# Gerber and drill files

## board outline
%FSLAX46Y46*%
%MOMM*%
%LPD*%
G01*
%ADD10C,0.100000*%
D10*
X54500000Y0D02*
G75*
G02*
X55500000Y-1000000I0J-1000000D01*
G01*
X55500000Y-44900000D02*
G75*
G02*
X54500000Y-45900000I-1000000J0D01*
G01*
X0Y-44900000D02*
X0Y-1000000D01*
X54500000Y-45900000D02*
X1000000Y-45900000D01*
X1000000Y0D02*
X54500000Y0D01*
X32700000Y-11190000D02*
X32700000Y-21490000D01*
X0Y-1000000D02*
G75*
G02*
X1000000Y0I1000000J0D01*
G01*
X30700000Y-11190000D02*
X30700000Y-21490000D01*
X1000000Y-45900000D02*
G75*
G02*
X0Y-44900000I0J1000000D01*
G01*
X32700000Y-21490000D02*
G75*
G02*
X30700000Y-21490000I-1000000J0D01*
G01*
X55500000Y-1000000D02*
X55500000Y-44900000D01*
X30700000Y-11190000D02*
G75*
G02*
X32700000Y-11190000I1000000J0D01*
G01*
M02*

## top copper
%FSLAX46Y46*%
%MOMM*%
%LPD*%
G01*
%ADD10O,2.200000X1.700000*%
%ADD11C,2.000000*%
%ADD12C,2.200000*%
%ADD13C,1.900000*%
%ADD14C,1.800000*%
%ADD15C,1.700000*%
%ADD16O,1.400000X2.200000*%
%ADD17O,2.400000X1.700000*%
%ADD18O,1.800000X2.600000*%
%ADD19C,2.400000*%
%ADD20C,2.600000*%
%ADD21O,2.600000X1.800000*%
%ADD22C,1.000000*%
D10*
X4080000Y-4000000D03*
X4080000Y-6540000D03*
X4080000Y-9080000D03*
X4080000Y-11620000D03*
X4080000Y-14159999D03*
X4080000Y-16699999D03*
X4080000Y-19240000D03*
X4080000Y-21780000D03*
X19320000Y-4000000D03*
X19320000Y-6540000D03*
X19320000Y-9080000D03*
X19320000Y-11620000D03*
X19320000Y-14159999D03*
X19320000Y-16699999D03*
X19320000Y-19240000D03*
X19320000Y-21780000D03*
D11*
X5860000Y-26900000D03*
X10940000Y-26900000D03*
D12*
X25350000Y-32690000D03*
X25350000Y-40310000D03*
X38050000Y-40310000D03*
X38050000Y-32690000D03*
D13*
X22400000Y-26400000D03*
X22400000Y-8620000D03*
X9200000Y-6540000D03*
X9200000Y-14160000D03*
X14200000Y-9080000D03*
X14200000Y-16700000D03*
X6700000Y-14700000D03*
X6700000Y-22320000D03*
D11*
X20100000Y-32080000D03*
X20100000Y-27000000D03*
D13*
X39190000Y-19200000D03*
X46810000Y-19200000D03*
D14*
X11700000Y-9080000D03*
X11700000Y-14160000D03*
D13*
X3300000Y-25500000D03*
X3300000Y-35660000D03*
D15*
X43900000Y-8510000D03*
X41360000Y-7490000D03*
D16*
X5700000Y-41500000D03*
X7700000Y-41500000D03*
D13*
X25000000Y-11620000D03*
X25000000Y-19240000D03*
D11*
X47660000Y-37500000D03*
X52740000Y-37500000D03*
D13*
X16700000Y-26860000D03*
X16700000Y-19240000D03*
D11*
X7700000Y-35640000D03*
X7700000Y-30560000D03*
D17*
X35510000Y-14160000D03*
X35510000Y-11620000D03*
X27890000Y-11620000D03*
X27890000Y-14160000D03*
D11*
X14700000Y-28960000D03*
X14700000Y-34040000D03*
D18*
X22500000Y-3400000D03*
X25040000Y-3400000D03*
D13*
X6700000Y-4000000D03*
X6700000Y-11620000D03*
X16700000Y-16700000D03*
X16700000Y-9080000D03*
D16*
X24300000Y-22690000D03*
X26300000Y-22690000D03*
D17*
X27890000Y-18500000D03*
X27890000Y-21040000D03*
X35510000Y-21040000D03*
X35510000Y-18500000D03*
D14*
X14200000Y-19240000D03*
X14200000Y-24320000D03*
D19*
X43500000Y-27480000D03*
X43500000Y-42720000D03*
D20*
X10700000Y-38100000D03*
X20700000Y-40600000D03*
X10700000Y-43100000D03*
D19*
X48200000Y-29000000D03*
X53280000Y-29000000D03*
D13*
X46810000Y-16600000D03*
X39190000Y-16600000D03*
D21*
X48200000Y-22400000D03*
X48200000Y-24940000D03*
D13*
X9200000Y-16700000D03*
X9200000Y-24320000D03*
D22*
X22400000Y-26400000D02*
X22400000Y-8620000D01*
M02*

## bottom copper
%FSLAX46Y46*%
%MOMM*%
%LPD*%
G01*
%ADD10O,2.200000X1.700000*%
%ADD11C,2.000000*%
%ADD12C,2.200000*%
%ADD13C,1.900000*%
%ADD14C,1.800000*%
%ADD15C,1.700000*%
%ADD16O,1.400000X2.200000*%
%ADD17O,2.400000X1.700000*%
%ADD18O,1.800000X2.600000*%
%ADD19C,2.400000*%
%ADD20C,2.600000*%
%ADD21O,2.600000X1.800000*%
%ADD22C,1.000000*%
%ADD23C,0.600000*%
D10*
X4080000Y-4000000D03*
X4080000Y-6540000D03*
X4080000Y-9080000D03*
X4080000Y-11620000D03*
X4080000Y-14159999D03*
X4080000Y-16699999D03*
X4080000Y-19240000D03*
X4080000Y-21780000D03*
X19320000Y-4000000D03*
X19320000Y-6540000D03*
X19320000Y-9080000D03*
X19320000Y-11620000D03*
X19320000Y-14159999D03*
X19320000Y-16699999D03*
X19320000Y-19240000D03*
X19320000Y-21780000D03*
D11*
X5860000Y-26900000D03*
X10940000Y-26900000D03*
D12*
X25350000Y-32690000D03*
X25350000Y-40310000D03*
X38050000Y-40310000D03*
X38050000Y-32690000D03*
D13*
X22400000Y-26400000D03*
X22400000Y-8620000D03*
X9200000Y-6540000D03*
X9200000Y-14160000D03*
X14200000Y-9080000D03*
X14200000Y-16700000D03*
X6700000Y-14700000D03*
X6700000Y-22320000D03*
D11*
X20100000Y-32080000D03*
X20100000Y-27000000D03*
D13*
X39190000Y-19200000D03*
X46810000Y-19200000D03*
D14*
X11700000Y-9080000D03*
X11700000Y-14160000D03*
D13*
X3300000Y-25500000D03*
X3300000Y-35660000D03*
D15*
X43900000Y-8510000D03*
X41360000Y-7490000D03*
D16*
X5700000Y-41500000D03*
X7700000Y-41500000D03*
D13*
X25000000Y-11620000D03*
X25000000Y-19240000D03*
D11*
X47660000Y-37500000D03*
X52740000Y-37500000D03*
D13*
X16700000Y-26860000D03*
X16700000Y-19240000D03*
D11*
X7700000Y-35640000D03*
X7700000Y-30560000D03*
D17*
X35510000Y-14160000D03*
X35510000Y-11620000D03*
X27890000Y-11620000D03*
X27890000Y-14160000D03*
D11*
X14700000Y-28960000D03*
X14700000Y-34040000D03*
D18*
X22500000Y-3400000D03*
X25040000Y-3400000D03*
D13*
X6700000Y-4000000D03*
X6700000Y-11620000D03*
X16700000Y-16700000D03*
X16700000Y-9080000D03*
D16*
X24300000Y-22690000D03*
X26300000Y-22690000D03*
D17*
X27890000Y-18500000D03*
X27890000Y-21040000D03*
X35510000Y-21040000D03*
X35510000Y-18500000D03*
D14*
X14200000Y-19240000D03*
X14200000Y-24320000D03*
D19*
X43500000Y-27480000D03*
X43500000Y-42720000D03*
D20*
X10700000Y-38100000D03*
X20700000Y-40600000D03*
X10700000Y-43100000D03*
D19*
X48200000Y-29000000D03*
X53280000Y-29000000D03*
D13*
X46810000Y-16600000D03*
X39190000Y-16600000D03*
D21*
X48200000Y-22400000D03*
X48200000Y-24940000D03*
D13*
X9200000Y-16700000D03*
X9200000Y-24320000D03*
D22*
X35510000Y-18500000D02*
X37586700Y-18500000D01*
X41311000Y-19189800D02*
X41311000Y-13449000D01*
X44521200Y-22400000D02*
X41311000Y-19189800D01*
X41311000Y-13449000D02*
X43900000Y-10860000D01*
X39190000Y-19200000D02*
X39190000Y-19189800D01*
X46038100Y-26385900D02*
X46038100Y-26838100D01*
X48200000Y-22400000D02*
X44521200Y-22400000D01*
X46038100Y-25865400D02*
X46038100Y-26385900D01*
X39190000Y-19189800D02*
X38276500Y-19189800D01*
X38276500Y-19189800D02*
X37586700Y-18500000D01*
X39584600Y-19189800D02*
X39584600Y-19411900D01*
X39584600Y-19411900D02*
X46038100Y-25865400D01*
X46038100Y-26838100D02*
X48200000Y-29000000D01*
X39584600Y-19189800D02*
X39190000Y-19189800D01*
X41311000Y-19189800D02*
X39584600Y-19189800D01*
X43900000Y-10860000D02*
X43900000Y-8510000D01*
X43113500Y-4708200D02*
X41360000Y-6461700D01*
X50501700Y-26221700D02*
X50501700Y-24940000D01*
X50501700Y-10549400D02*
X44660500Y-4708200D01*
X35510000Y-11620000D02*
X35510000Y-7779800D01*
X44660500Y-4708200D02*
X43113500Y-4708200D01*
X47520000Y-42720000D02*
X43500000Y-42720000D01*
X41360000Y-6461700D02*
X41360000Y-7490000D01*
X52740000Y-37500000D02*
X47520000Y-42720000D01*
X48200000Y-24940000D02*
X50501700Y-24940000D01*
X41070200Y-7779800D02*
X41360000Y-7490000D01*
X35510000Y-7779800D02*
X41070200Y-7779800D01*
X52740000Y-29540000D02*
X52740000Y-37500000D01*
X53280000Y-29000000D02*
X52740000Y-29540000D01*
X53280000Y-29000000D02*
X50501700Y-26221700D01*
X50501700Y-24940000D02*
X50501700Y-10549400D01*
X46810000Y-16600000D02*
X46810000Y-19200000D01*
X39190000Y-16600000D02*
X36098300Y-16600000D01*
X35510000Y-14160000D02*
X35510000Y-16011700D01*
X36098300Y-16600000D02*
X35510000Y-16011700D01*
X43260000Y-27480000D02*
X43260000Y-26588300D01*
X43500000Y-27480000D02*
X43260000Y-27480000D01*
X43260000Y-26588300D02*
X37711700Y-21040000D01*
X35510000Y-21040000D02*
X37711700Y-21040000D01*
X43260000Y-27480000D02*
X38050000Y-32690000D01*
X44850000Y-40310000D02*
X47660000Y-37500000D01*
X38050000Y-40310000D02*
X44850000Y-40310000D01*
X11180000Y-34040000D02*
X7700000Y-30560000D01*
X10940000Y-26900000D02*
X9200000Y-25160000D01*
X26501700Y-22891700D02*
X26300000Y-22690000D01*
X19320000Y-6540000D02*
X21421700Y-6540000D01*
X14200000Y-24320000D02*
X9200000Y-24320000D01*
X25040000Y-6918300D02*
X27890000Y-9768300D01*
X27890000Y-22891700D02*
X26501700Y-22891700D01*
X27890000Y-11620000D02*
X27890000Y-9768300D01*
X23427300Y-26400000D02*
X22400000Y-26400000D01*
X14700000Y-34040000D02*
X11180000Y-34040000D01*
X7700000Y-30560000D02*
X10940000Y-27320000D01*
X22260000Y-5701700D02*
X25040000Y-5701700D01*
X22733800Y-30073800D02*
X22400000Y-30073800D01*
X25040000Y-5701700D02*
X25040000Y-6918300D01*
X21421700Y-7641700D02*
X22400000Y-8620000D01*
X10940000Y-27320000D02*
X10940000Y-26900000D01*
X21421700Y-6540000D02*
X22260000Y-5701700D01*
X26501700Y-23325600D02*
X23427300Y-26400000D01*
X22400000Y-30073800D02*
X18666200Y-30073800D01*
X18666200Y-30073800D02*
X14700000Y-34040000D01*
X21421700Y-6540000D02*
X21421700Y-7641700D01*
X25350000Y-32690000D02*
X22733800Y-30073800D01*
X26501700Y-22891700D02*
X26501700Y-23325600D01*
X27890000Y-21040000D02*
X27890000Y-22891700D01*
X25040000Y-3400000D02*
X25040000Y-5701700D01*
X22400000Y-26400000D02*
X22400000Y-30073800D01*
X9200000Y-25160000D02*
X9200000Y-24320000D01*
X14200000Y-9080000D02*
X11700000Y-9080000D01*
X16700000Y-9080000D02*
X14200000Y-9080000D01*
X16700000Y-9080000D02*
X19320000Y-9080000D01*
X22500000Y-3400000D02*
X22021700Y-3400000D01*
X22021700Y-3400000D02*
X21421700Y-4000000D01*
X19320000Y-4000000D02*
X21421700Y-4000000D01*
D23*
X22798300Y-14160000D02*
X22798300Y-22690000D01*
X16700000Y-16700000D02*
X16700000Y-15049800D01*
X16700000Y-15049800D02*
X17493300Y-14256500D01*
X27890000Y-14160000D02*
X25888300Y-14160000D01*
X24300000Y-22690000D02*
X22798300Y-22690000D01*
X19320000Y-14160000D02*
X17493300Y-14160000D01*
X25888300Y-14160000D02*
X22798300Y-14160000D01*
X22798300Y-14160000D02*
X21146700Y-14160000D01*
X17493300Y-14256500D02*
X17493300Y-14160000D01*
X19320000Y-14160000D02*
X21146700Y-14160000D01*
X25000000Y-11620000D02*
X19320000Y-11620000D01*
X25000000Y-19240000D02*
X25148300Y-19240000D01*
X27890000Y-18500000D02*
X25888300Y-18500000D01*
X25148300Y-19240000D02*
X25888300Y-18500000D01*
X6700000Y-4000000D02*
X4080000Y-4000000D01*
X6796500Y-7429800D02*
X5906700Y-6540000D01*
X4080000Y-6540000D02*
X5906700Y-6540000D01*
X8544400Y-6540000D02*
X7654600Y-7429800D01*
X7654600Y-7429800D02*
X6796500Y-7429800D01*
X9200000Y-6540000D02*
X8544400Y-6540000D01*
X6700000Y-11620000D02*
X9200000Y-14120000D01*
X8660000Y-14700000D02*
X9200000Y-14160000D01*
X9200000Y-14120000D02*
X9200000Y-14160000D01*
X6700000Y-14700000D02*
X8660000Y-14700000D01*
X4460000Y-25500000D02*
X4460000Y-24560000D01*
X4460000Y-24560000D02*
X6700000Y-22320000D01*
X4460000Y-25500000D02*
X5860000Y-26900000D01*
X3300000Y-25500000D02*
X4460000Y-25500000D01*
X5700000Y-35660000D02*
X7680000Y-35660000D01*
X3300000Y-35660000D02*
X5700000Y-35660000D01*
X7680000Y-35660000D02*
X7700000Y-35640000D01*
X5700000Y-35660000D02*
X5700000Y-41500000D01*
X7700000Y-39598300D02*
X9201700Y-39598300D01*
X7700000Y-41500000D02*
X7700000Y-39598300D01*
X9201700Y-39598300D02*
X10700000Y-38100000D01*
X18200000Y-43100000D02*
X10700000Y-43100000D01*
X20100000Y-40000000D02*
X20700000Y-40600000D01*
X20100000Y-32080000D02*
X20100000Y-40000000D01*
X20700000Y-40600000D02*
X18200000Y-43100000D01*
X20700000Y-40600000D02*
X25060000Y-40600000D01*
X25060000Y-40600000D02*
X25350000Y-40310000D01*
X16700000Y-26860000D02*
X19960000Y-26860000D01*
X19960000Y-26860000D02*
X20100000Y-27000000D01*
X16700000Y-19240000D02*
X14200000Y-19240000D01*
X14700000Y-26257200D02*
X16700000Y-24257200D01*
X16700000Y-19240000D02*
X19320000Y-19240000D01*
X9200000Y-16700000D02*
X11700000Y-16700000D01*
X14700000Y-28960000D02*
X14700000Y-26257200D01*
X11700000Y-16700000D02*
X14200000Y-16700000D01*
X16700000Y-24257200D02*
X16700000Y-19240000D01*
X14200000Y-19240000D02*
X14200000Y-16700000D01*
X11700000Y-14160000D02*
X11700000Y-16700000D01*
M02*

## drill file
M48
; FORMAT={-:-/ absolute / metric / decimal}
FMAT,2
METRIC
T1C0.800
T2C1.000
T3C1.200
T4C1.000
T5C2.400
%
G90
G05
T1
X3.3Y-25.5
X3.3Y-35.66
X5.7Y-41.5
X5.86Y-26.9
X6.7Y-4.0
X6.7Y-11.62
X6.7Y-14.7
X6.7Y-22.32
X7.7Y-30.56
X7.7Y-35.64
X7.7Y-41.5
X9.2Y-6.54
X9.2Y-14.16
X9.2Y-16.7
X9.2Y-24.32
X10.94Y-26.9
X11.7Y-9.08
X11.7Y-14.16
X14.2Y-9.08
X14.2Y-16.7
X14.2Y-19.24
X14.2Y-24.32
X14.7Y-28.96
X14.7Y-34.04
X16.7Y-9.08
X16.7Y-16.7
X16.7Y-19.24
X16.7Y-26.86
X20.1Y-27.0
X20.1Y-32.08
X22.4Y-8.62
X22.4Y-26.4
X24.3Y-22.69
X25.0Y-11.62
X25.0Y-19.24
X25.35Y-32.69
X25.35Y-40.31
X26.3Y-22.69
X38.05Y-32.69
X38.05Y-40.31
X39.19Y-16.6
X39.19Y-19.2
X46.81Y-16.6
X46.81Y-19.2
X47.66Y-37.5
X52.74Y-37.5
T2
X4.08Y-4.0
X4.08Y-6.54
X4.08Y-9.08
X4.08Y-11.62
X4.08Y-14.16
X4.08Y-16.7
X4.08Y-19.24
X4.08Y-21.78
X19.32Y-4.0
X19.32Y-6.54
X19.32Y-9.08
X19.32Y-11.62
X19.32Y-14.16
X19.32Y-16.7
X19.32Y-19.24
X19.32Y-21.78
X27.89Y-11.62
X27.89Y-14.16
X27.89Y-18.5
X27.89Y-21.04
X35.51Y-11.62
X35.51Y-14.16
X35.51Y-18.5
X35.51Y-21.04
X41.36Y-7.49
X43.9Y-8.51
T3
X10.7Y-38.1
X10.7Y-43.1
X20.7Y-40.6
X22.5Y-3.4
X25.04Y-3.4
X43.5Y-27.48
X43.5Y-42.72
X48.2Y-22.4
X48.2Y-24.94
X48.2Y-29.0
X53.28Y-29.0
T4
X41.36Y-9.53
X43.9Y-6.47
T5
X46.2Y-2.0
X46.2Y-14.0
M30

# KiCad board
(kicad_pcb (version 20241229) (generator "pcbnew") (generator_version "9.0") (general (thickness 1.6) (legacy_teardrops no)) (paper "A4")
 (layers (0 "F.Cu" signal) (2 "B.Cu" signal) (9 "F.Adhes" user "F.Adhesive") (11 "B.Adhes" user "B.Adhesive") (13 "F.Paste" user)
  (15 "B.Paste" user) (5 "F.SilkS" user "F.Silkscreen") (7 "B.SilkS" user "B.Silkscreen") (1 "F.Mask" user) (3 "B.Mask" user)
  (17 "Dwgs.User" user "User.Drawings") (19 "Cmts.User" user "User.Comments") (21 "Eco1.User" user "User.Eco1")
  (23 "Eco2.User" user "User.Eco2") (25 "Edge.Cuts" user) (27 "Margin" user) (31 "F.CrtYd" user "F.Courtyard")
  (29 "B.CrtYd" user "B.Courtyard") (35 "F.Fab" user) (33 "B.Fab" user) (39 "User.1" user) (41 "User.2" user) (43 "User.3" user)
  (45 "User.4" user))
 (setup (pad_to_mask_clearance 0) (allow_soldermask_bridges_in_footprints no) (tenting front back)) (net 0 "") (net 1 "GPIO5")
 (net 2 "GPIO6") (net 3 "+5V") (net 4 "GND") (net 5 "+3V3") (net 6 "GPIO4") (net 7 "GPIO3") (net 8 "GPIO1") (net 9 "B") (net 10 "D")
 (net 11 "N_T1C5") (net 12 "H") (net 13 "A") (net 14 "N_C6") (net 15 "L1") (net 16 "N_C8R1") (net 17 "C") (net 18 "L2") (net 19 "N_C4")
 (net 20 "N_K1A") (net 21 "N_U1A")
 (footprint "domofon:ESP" (layer "F.Cu") (at 11.7 12.89)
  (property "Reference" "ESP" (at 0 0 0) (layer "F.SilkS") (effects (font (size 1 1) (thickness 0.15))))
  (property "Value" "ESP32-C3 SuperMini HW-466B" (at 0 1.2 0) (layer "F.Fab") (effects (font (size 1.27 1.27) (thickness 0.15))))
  (pad "L1" thru_hole oval (at -7.62 -8.89) (size 2.2 1.7) (drill 1) (layers "B.Cu" "B.Mask") (remove_unused_layers no) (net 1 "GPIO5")
   (thermal_bridge_angle 45))
  (pad "L2" thru_hole oval (at -7.62 -6.35) (size 2.2 1.7) (drill 1) (layers "B.Cu" "B.Mask") (remove_unused_layers no) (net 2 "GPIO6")
   (thermal_bridge_angle 45))
  (pad "L3" thru_hole oval (at -7.62 -3.81) (size 2.2 1.7) (drill 1) (layers "B.Cu" "B.Mask") (remove_unused_layers no)
   (thermal_bridge_angle 45))
  (pad "L4" thru_hole oval (at -7.62 -1.27) (size 2.2 1.7) (drill 1) (layers "B.Cu" "B.Mask") (remove_unused_layers no)
   (thermal_bridge_angle 45))
  (pad "L5" thru_hole oval (at -7.62 1.269999) (size 2.2 1.7) (drill 1) (layers "B.Cu" "B.Mask") (remove_unused_layers no)
   (thermal_bridge_angle 45))
  (pad "L6" thru_hole oval (at -7.62 3.809999) (size 2.2 1.7) (drill 1) (layers "B.Cu" "B.Mask") (remove_unused_layers no)
   (thermal_bridge_angle 45))
  (pad "L7" thru_hole oval (at -7.62 6.35) (size 2.2 1.7) (drill 1) (layers "B.Cu" "B.Mask") (remove_unused_layers no)
   (thermal_bridge_angle 45))
  (pad "L8" thru_hole oval (at -7.62 8.89) (size 2.2 1.7) (drill 1) (layers "B.Cu" "B.Mask") (remove_unused_layers no)
   (thermal_bridge_angle 45))
  (pad "R1" thru_hole oval (at 7.62 -8.89) (size 2.2 1.7) (drill 1) (layers "B.Cu" "B.Mask") (remove_unused_layers no) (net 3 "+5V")
   (thermal_bridge_angle 45))
  (pad "R2" thru_hole oval (at 7.62 -6.35) (size 2.2 1.7) (drill 1) (layers "B.Cu" "B.Mask") (remove_unused_layers no) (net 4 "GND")
   (thermal_bridge_angle 45))
  (pad "R3" thru_hole oval (at 7.62 -3.81) (size 2.2 1.7) (drill 1) (layers "B.Cu" "B.Mask") (remove_unused_layers no) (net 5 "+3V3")
   (thermal_bridge_angle 45))
  (pad "R4" thru_hole oval (at 7.62 -1.27) (size 2.2 1.7) (drill 1) (layers "B.Cu" "B.Mask") (remove_unused_layers no) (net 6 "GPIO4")
   (thermal_bridge_angle 45))
  (pad "R5" thru_hole oval (at 7.62 1.269999) (size 2.2 1.7) (drill 1) (layers "B.Cu" "B.Mask") (remove_unused_layers no) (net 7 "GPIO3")
   (thermal_bridge_angle 45))
  (pad "R6" thru_hole oval (at 7.62 3.809999) (size 2.2 1.7) (drill 1) (layers "B.Cu" "B.Mask") (remove_unused_layers no)
   (thermal_bridge_angle 45))
  (pad "R7" thru_hole oval (at 7.62 6.35) (size 2.2 1.7) (drill 1) (layers "B.Cu" "B.Mask") (remove_unused_layers no) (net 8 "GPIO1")
   (thermal_bridge_angle 45))
  (pad "R8" thru_hole oval (at 7.62 8.89) (size 2.2 1.7) (drill 1) (layers "B.Cu" "B.Mask") (remove_unused_layers no)
   (thermal_bridge_angle 45)))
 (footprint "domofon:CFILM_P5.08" (layer "F.Cu") (at 8.4 26.9)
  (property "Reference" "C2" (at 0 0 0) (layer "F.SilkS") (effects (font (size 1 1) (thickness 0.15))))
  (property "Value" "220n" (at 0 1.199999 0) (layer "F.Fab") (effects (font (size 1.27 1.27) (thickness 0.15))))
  (pad "1" thru_hole circle (at -2.54 0) (size 2 2) (drill 0.8) (layers "B.Cu" "B.Mask") (remove_unused_layers no) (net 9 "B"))
  (pad "2" thru_hole circle (at 2.54 0) (size 2 2) (drill 0.8) (layers "B.Cu" "B.Mask") (remove_unused_layers no) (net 4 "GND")))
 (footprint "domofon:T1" (layer "F.Cu") (at 31.7 36.5)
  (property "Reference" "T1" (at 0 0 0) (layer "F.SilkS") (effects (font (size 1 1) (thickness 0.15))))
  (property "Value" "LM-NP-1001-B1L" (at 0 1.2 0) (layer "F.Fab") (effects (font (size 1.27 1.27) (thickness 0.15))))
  (pad "1" thru_hole circle (at -6.35 -3.81) (size 2.2 2.2) (drill 0.8) (layers "B.Cu" "B.Mask") (remove_unused_layers no) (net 4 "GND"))
  (pad "4" thru_hole circle (at -6.35 3.81) (size 2.2 2.2) (drill 0.8) (layers "B.Cu" "B.Mask") (remove_unused_layers no) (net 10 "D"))
  (pad "5" thru_hole circle (at 6.35 3.81) (size 2.2 2.2) (drill 0.8) (layers "B.Cu" "B.Mask") (remove_unused_layers no) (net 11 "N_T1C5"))
  (pad "8" thru_hole circle (at 6.35 -3.81) (size 2.2 2.2) (drill 0.8) (layers "B.Cu" "B.Mask") (remove_unused_layers no) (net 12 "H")))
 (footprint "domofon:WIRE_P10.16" (layer "F.Cu") (at 22.4 17.51 90)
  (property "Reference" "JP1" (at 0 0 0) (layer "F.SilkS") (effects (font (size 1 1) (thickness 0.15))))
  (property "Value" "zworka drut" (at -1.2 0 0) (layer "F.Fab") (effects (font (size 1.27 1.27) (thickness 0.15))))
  (pad "1" thru_hole circle (at -8.89 0 90) (size 1.9 1.9) (drill 0.8) (layers "*.Cu" "B.Mask") (remove_unused_layers no) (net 4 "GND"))
  (pad "2" thru_hole circle (at 8.89 0 90) (size 1.9 1.9) (drill 0.8) (layers "*.Cu" "B.Mask") (remove_unused_layers no) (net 4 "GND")))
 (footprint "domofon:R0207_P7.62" (layer "F.Cu") (at 9.2 10.35 -90)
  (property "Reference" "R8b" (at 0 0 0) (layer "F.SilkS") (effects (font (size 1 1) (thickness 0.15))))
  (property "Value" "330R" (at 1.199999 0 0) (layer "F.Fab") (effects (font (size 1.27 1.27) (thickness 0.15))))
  (pad "1" thru_hole circle (at -3.81 0 270) (size 1.9 1.9) (drill 0.8) (layers "B.Cu" "B.Mask") (remove_unused_layers no) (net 2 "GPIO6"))
  (pad "2" thru_hole circle (at 3.81 0 270) (size 1.9 1.9) (drill 0.8) (layers "B.Cu" "B.Mask") (remove_unused_layers no) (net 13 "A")))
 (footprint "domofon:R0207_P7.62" (layer "F.Cu") (at 14.2 12.89 -90)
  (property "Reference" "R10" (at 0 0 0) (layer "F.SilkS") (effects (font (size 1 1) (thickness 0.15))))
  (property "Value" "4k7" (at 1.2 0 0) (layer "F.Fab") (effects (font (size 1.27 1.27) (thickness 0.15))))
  (pad "1" thru_hole circle (at -3.81 0 270) (size 1.9 1.9) (drill 0.8) (layers "B.Cu" "B.Mask") (remove_unused_layers no) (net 5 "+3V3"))
  (pad "2" thru_hole circle (at 3.81 0 270) (size 1.9 1.9) (drill 0.8) (layers "B.Cu" "B.Mask") (remove_unused_layers no) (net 8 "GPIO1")))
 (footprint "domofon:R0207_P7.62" (layer "F.Cu") (at 6.7 18.51 -90)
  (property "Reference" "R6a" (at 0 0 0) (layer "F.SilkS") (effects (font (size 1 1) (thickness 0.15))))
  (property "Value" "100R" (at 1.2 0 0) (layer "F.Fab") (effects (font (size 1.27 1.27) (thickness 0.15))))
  (pad "1" thru_hole circle (at -3.81 0 270) (size 1.9 1.9) (drill 0.8) (layers "B.Cu" "B.Mask") (remove_unused_layers no) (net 13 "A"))
  (pad "2" thru_hole circle (at 3.81 0 270) (size 1.9 1.9) (drill 0.8) (layers "B.Cu" "B.Mask") (remove_unused_layers no) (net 9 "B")))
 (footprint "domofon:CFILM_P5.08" (layer "F.Cu") (at 20.1 29.54 90)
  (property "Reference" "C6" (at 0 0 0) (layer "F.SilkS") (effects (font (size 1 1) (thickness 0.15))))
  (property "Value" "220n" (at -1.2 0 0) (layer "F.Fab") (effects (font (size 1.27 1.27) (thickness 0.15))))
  (pad "1" thru_hole circle (at -2.54 0 90) (size 2 2) (drill 0.8) (layers "B.Cu" "B.Mask") (remove_unused_layers no) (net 10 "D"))
  (pad "2" thru_hole circle (at 2.54 0 90) (size 2 2) (drill 0.8) (layers "B.Cu" "B.Mask") (remove_unused_layers no) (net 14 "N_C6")))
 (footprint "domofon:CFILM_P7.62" (layer "F.Cu") (at 43 19.2)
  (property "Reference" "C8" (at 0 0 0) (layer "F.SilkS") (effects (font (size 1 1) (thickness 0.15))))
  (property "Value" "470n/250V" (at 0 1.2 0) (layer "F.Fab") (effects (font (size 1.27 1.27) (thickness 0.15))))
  (pad "1" thru_hole circle (at -3.81 0) (size 1.9 1.9) (drill 0.8) (layers "B.Cu" "B.Mask") (remove_unused_layers no) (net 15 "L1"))
  (pad "2" thru_hole circle (at 3.81 0) (size 1.9 1.9) (drill 0.8) (layers "B.Cu" "B.Mask") (remove_unused_layers no) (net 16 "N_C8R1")))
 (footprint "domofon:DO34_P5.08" (layer "F.Cu") (at 11.7 11.62 -90)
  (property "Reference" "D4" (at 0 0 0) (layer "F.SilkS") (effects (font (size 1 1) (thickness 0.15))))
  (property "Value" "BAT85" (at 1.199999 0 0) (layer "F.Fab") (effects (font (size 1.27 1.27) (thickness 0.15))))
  (pad "1" thru_hole circle (at -2.54 0 270) (size 1.8 1.8) (drill 0.8) (layers "B.Cu" "B.Mask") (remove_unused_layers no) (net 5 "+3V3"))
  (pad "2" thru_hole circle (at 2.54 0 270) (size 1.8 1.8) (drill 0.8) (layers "B.Cu" "B.Mask") (remove_unused_layers no) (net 8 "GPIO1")))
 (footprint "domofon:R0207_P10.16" (layer "F.Cu") (at 3.3 30.58 -90)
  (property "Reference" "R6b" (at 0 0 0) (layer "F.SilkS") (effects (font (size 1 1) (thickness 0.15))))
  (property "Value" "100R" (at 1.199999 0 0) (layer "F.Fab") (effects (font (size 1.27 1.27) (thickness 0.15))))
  (pad "1" thru_hole circle (at -5.08 0 270) (size 1.9 1.9) (drill 0.8) (layers "B.Cu" "B.Mask") (remove_unused_layers no) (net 9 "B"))
  (pad "2" thru_hole circle (at 5.08 0 270) (size 1.9 1.9) (drill 0.8) (layers "B.Cu" "B.Mask") (remove_unused_layers no) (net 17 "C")))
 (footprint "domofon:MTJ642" (layer "F.Cu") (at 46.2 8)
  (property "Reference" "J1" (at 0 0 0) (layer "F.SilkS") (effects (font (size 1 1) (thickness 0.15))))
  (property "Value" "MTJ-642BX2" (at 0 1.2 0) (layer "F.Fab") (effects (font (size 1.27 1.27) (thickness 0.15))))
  (pad "" np_thru_hole circle (at -4.84 1.53) (size 1 1) (drill 1) (layers "B.Cu" "B.Mask"))
  (pad "" np_thru_hole circle (at -2.3 -1.53) (size 1 1) (drill 1) (layers "B.Cu" "B.Mask"))
  (pad "" np_thru_hole circle (at 0 -6) (size 2.4 2.4) (drill 2.4) (layers "B.Cu" "B.Mask"))
  (pad "" np_thru_hole circle (at 0 6) (size 2.4 2.4) (drill 2.4) (layers "B.Cu" "B.Mask"))
  (pad "2" thru_hole circle (at -2.3 0.51) (size 1.7 1.7) (drill 1) (layers "B.Cu" "B.Mask") (remove_unused_layers no) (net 15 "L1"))
  (pad "3" thru_hole circle (at -4.84 -0.51) (size 1.7 1.7) (drill 1) (layers "B.Cu" "B.Mask") (remove_unused_layers no) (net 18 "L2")))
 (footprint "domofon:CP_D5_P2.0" (layer "F.Cu") (at 6.7 41.5)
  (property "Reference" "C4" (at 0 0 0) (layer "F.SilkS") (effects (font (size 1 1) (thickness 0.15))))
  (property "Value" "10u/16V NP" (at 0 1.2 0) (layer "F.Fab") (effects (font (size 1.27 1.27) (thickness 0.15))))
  (pad "1" thru_hole oval (at -1 0) (size 1.4 2.2) (drill 0.8) (layers "B.Cu" "B.Mask") (remove_unused_layers no) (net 17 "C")
   (thermal_bridge_angle 45))
  (pad "2" thru_hole oval (at 1 0) (size 1.4 2.2) (drill 0.8) (layers "B.Cu" "B.Mask") (remove_unused_layers no) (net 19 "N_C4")
   (thermal_bridge_angle 45)))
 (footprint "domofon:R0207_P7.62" (layer "F.Cu") (at 25 15.43 -90)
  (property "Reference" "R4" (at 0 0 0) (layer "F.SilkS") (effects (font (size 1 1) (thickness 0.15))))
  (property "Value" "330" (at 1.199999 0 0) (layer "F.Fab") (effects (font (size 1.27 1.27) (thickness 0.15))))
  (pad "1" thru_hole circle (at -3.81 0 270) (size 1.9 1.9) (drill 0.8) (layers "B.Cu" "B.Mask") (remove_unused_layers no) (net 6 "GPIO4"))
  (pad "2" thru_hole circle (at 3.81 0 270) (size 1.9 1.9) (drill 0.8) (layers "B.Cu" "B.Mask") (remove_unused_layers no) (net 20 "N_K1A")))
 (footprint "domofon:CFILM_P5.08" (layer "F.Cu") (at 50.2 37.5)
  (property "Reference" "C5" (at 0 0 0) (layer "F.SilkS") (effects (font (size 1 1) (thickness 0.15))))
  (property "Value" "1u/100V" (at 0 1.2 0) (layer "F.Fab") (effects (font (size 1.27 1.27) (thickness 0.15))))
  (pad "1" thru_hole circle (at -2.54 0) (size 2 2) (drill 0.8) (layers "B.Cu" "B.Mask") (remove_unused_layers no) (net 11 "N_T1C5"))
  (pad "2" thru_hole circle (at 2.54 0) (size 2 2) (drill 0.8) (layers "B.Cu" "B.Mask") (remove_unused_layers no) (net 18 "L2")))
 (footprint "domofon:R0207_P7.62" (layer "F.Cu") (at 16.7 23.05 90)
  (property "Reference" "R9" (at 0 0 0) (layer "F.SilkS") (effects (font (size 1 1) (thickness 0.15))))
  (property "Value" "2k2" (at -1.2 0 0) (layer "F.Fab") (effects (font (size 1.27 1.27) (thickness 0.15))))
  (pad "1" thru_hole circle (at -3.81 0 90) (size 1.9 1.9) (drill 0.8) (layers "B.Cu" "B.Mask") (remove_unused_layers no) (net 14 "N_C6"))
  (pad "2" thru_hole circle (at 3.81 0 90) (size 1.9 1.9) (drill 0.8) (layers "B.Cu" "B.Mask") (remove_unused_layers no) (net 8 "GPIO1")))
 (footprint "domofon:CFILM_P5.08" (layer "F.Cu") (at 7.7 33.1 90)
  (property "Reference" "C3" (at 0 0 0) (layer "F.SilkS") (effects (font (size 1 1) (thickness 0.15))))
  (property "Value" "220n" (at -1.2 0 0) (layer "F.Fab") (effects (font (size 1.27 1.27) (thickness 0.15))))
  (pad "1" thru_hole circle (at -2.54 0 90) (size 2 2) (drill 0.8) (layers "B.Cu" "B.Mask") (remove_unused_layers no) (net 17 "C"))
  (pad "2" thru_hole circle (at 2.54 0 90) (size 2 2) (drill 0.8) (layers "B.Cu" "B.Mask") (remove_unused_layers no) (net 4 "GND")))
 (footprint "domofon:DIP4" (layer "F.Cu") (at 31.7 12.89 180)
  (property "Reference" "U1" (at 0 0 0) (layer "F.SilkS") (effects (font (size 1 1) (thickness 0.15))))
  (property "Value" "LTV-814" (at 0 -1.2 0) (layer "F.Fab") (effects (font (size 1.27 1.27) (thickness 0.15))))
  (pad "1" thru_hole oval (at -3.81 -1.27 180) (size 2.4 1.7) (drill 1) (layers "B.Cu" "B.Mask") (remove_unused_layers no) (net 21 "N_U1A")
   (thermal_bridge_angle 45))
  (pad "2" thru_hole oval (at -3.81 1.27 180) (size 2.4 1.7) (drill 1) (layers "B.Cu" "B.Mask") (remove_unused_layers no) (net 18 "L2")
   (thermal_bridge_angle 45))
  (pad "3" thru_hole oval (at 3.81 1.27 180) (size 2.4 1.7) (drill 1) (layers "B.Cu" "B.Mask") (remove_unused_layers no) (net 4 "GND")
   (thermal_bridge_angle 45))
  (pad "4" thru_hole oval (at 3.81 -1.27 180) (size 2.4 1.7) (drill 1) (layers "B.Cu" "B.Mask") (remove_unused_layers no) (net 7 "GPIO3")
   (thermal_bridge_angle 45)))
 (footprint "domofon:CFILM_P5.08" (layer "F.Cu") (at 14.7 31.5 -90)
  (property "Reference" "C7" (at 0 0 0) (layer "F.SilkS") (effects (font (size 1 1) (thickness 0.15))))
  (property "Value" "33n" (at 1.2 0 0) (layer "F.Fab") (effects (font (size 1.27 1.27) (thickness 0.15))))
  (pad "1" thru_hole circle (at -2.54 0 270) (size 2 2) (drill 0.8) (layers "B.Cu" "B.Mask") (remove_unused_layers no) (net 8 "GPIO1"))
  (pad "2" thru_hole circle (at 2.54 0 270) (size 2 2) (drill 0.8) (layers "B.Cu" "B.Mask") (remove_unused_layers no) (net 4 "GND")))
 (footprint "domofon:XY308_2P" (layer "F.Cu") (at 22.5 3.4 90)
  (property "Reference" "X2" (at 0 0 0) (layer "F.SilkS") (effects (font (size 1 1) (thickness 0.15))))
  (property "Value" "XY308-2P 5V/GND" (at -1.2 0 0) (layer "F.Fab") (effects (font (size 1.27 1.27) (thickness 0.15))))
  (pad "1" thru_hole oval (at 0 0 90) (size 2.6 1.8) (drill 1.2) (layers "B.Cu" "B.Mask") (remove_unused_layers no) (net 3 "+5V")
   (thermal_bridge_angle 45))
  (pad "2" thru_hole oval (at 0 2.54 90) (size 2.6 1.8) (drill 1.2) (layers "B.Cu" "B.Mask") (remove_unused_layers no) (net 4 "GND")
   (thermal_bridge_angle 45)))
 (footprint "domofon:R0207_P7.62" (layer "F.Cu") (at 6.7 7.81 -90)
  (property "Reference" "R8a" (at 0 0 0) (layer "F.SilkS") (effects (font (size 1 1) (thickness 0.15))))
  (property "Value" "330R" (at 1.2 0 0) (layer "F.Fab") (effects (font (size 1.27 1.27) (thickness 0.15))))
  (pad "1" thru_hole circle (at -3.81 0 270) (size 1.9 1.9) (drill 0.8) (layers "B.Cu" "B.Mask") (remove_unused_layers no) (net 1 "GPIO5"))
  (pad "2" thru_hole circle (at 3.81 0 270) (size 1.9 1.9) (drill 0.8) (layers "B.Cu" "B.Mask") (remove_unused_layers no) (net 13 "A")))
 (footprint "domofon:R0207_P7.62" (layer "F.Cu") (at 16.7 12.89 90)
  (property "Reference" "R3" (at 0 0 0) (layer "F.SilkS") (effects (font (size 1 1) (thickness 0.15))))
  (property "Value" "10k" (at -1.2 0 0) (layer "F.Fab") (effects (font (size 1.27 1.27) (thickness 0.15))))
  (pad "1" thru_hole circle (at -3.81 0 90) (size 1.9 1.9) (drill 0.8) (layers "B.Cu" "B.Mask") (remove_unused_layers no) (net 7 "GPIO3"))
  (pad "2" thru_hole circle (at 3.81 0 90) (size 1.9 1.9) (drill 0.8) (layers "B.Cu" "B.Mask") (remove_unused_layers no) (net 5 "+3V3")))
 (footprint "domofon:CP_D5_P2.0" (layer "F.Cu") (at 25.3 22.69)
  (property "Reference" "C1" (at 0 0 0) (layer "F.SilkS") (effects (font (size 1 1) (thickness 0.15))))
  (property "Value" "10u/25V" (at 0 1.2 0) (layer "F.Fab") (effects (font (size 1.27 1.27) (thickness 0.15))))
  (pad "1" thru_hole oval (at -1 0) (size 1.4 2.2) (drill 0.8) (layers "B.Cu" "B.Mask") (remove_unused_layers no) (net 7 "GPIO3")
   (thermal_bridge_angle 45))
  (pad "2" thru_hole oval (at 1 0) (size 1.4 2.2) (drill 0.8) (layers "B.Cu" "B.Mask") (remove_unused_layers no) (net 4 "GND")
   (thermal_bridge_angle 45)))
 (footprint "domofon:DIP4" (layer "F.Cu") (at 31.7 19.77)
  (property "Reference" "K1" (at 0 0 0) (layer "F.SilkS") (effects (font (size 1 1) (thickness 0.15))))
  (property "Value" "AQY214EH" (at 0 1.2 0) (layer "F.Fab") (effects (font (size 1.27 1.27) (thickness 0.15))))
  (pad "1" thru_hole oval (at -3.81 -1.27) (size 2.4 1.7) (drill 1) (layers "B.Cu" "B.Mask") (remove_unused_layers no) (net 20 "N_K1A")
   (thermal_bridge_angle 45))
  (pad "2" thru_hole oval (at -3.81 1.27) (size 2.4 1.7) (drill 1) (layers "B.Cu" "B.Mask") (remove_unused_layers no) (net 4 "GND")
   (thermal_bridge_angle 45))
  (pad "3" thru_hole oval (at 3.81 1.27) (size 2.4 1.7) (drill 1) (layers "B.Cu" "B.Mask") (remove_unused_layers no) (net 12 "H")
   (thermal_bridge_angle 45))
  (pad "4" thru_hole oval (at 3.81 -1.27) (size 2.4 1.7) (drill 1) (layers "B.Cu" "B.Mask") (remove_unused_layers no) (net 15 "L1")
   (thermal_bridge_angle 45)))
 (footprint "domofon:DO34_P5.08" (layer "F.Cu") (at 14.2 21.78 -90)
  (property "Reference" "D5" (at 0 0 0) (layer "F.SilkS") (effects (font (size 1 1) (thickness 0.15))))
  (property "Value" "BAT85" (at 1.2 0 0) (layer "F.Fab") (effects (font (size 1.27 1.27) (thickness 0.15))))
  (pad "1" thru_hole circle (at -2.54 0 270) (size 1.8 1.8) (drill 0.8) (layers "B.Cu" "B.Mask") (remove_unused_layers no) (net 8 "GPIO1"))
  (pad "2" thru_hole circle (at 2.54 0 270) (size 1.8 1.8) (drill 0.8) (layers "B.Cu" "B.Mask") (remove_unused_layers no) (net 4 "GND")))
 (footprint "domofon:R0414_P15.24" (layer "F.Cu") (at 43.5 35.1 -90)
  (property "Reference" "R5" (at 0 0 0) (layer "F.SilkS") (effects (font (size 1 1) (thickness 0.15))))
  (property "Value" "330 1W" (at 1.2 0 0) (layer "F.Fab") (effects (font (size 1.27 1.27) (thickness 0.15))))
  (pad "1" thru_hole circle (at -7.62 0 270) (size 2.4 2.4) (drill 1.2) (layers "B.Cu" "B.Mask") (remove_unused_layers no) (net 12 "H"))
  (pad "2" thru_hole circle (at 7.62 0 270) (size 2.4 2.4) (drill 1.2) (layers "B.Cu" "B.Mask") (remove_unused_layers no) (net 18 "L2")))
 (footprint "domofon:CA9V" (layer "F.Cu") (at 10.7 40.6 -90)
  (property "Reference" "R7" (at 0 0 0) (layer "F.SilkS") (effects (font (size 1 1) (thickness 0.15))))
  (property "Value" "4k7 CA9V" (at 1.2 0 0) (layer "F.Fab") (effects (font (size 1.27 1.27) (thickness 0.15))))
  (pad "1" thru_hole circle (at -2.5 0 270) (size 2.6 2.6) (drill 1.2) (layers "B.Cu" "B.Mask") (remove_unused_layers no) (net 19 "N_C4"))
  (pad "2" thru_hole circle (at 0 -10 270) (size 2.6 2.6) (drill 1.2) (layers "B.Cu" "B.Mask") (remove_unused_layers no) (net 10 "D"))
  (pad "3" thru_hole circle (at 2.5 0 270) (size 2.6 2.6) (drill 1.2) (layers "B.Cu" "B.Mask") (remove_unused_layers no) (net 10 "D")))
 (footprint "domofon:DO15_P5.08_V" (layer "F.Cu") (at 50.74 29)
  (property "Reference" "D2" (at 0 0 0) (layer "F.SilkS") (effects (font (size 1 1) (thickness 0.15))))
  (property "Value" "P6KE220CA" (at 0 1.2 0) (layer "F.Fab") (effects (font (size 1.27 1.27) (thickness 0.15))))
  (pad "1" thru_hole circle (at -2.54 0) (size 2.4 2.4) (drill 1.2) (layers "B.Cu" "B.Mask") (remove_unused_layers no) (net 15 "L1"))
  (pad "2" thru_hole circle (at 2.54 0) (size 2.4 2.4) (drill 1.2) (layers "B.Cu" "B.Mask") (remove_unused_layers no) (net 18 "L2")))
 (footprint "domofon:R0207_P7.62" (layer "F.Cu") (at 43 16.6 180)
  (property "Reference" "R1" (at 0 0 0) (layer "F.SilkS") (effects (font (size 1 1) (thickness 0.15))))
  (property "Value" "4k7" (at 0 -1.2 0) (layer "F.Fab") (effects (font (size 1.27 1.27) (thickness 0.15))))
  (pad "1" thru_hole circle (at -3.81 0 180) (size 1.9 1.9) (drill 0.8) (layers "B.Cu" "B.Mask") (remove_unused_layers no) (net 16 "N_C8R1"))
  (pad "2" thru_hole circle (at 3.81 0 180) (size 1.9 1.9) (drill 0.8) (layers "B.Cu" "B.Mask") (remove_unused_layers no) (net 21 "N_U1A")))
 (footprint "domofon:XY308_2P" (layer "F.Cu") (at 48.2 22.4)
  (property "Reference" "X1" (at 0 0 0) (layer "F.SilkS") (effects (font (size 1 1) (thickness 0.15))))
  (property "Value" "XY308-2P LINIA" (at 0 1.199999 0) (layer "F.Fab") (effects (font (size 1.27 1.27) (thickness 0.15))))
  (pad "1" thru_hole oval (at 0 0) (size 2.6 1.8) (drill 1.2) (layers "B.Cu" "B.Mask") (remove_unused_layers no) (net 15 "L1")
   (thermal_bridge_angle 45))
  (pad "2" thru_hole oval (at 0 2.54) (size 2.6 1.8) (drill 1.2) (layers "B.Cu" "B.Mask") (remove_unused_layers no) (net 18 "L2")
   (thermal_bridge_angle 45)))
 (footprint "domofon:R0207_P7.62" (layer "F.Cu") (at 9.2 20.51 -90)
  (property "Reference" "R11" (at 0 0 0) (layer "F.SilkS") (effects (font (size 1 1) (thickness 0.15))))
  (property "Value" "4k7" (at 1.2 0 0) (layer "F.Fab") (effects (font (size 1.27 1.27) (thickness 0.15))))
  (pad "1" thru_hole circle (at -3.81 0 270) (size 1.9 1.9) (drill 0.8) (layers "B.Cu" "B.Mask") (remove_unused_layers no) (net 8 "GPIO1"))
  (pad "2" thru_hole circle (at 3.81 0 270) (size 1.9 1.9) (drill 0.8) (layers "B.Cu" "B.Mask") (remove_unused_layers no) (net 4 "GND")))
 (gr_arc (start 54.5 0) (mid 55.207107 0.292893) (end 55.5 1) (stroke (width 0.1) (type default)) (layer "Edge.Cuts"))
 (gr_arc (start 55.5 44.9) (mid 55.207107 45.607107) (end 54.5 45.9) (stroke (width 0.1) (type default)) (layer "Edge.Cuts"))
 (gr_line (start 0 44.9) (end 0 1) (stroke (width 0.1) (type default)) (layer "Edge.Cuts"))
 (gr_line (start 54.5 45.9) (end 1 45.9) (stroke (width 0.1) (type default)) (layer "Edge.Cuts"))
 (gr_line (start 1 0) (end 54.5 0) (stroke (width 0.1) (type default)) (layer "Edge.Cuts"))
 (gr_line (start 32.7 11.19) (end 32.7 21.49) (stroke (width 0.1) (type default)) (layer "Edge.Cuts"))
 (gr_arc (start 0 1) (mid 0.292893 0.292893) (end 1 0) (stroke (width 0.1) (type default)) (layer "Edge.Cuts"))
 (gr_line (start 30.7 11.19) (end 30.7 21.49) (stroke (width 0.1) (type default)) (layer "Edge.Cuts"))
 (gr_arc (start 1 45.9) (mid 0.292893 45.607107) (end 0 44.9) (stroke (width 0.1) (type default)) (layer "Edge.Cuts"))
 (gr_arc (start 32.7 21.49) (mid 31.7 22.49) (end 30.7 21.49) (stroke (width 0.1) (type default)) (layer "Edge.Cuts"))
 (gr_line (start 55.5 1) (end 55.5 44.9) (stroke (width 0.1) (type default)) (layer "Edge.Cuts"))
 (gr_arc (start 30.7 11.19) (mid 31.7 10.19) (end 32.7 11.19) (stroke (width 0.1) (type default)) (layer "Edge.Cuts"))
 (segment (start 35.51 18.5) (end 37.5867 18.5) (width 1) (layer "B.Cu") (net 15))
 (segment (start 41.311 19.1898) (end 41.311 13.449) (width 1) (layer "B.Cu") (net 15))
 (segment (start 44.5212 22.4) (end 41.311 19.1898) (width 1) (layer "B.Cu") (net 15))
 (segment (start 41.311 13.449) (end 43.9 10.86) (width 1) (layer "B.Cu") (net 15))
 (segment (start 39.19 19.2) (end 39.19 19.1898) (width 1) (layer "B.Cu") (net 15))
 (segment (start 46.0381 26.3859) (end 46.0381 26.8381) (width 1) (layer "B.Cu") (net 15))
 (segment (start 48.2 22.4) (end 44.5212 22.4) (width 1) (layer "B.Cu") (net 15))
 (segment (start 46.0381 25.8654) (end 46.0381 26.3859) (width 1) (layer "B.Cu") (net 15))
 (segment (start 39.19 19.1898) (end 38.2765 19.1898) (width 1) (layer "B.Cu") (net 15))
 (segment (start 38.2765 19.1898) (end 37.5867 18.5) (width 1) (layer "B.Cu") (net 15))
 (segment (start 39.5846 19.1898) (end 39.5846 19.4119) (width 1) (layer "B.Cu") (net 15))
 (segment (start 39.5846 19.4119) (end 46.0381 25.8654) (width 1) (layer "B.Cu") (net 15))
 (segment (start 46.0381 26.8381) (end 48.2 29) (width 1) (layer "B.Cu") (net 15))
 (segment (start 39.5846 19.1898) (end 39.19 19.1898) (width 1) (layer "B.Cu") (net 15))
 (segment (start 41.311 19.1898) (end 39.5846 19.1898) (width 1) (layer "B.Cu") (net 15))
 (segment (start 43.9 10.86) (end 43.9 8.51) (width 1) (layer "B.Cu") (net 15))
 (segment (start 43.1135 4.7082) (end 41.36 6.4617) (width 1) (layer "B.Cu") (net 18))
 (segment (start 50.5017 26.2217) (end 50.5017 24.94) (width 1) (layer "B.Cu") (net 18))
 (segment (start 50.5017 10.5494) (end 44.6605 4.7082) (width 1) (layer "B.Cu") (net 18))
 (segment (start 35.51 11.62) (end 35.51 7.7798) (width 1) (layer "B.Cu") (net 18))
 (segment (start 44.6605 4.7082) (end 43.1135 4.7082) (width 1) (layer "B.Cu") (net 18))
 (segment (start 47.52 42.72) (end 43.5 42.72) (width 1) (layer "B.Cu") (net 18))
 (segment (start 41.36 6.4617) (end 41.36 7.49) (width 1) (layer "B.Cu") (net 18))
 (segment (start 52.74 37.5) (end 47.52 42.72) (width 1) (layer "B.Cu") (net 18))
 (segment (start 48.2 24.94) (end 50.5017 24.94) (width 1) (layer "B.Cu") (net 18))
 (segment (start 41.0702 7.7798) (end 41.36 7.49) (width 1) (layer "B.Cu") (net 18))
 (segment (start 35.51 7.7798) (end 41.0702 7.7798) (width 1) (layer "B.Cu") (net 18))
 (segment (start 52.74 29.54) (end 52.74 37.5) (width 1) (layer "B.Cu") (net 18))
 (segment (start 53.28 29) (end 52.74 29.54) (width 1) (layer "B.Cu") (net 18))
 (segment (start 53.28 29) (end 50.5017 26.2217) (width 1) (layer "B.Cu") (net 18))
 (segment (start 50.5017 24.94) (end 50.5017 10.5494) (width 1) (layer "B.Cu") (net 18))
 (segment (start 46.81 16.6) (end 46.81 19.2) (width 1) (layer "B.Cu") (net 16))
 (segment (start 39.19 16.6) (end 36.0983 16.6) (width 1) (layer "B.Cu") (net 21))
 (segment (start 35.51 14.16) (end 35.51 16.0117) (width 1) (layer "B.Cu") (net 21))
 (segment (start 36.0983 16.6) (end 35.51 16.0117) (width 1) (layer "B.Cu") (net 21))
 (segment (start 43.26 27.48) (end 43.26 26.5883) (width 1) (layer "B.Cu") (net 12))
 (segment (start 43.5 27.48) (end 43.26 27.48) (width 1) (layer "B.Cu") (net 12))
 (segment (start 43.26 26.5883) (end 37.7117 21.04) (width 1) (layer "B.Cu") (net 12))
 (segment (start 35.51 21.04) (end 37.7117 21.04) (width 1) (layer "B.Cu") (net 12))
 (segment (start 43.26 27.48) (end 38.05 32.69) (width 1) (layer "B.Cu") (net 12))
 (segment (start 44.85 40.31) (end 47.66 37.5) (width 1) (layer "B.Cu") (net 11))
 (segment (start 38.05 40.31) (end 44.85 40.31) (width 1) (layer "B.Cu") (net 11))
 (segment (start 22.4 26.4) (end 22.4 8.62) (width 1) (layer "F.Cu") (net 4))
 (segment (start 11.18 34.04) (end 7.7 30.56) (width 1) (layer "B.Cu") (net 4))
 (segment (start 10.94 26.9) (end 9.2 25.16) (width 1) (layer "B.Cu") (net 4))
 (segment (start 26.5017 22.8917) (end 26.3 22.69) (width 1) (layer "B.Cu") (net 4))
 (segment (start 19.32 6.54) (end 21.4217 6.54) (width 1) (layer "B.Cu") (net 4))
 (segment (start 14.2 24.32) (end 9.2 24.32) (width 1) (layer "B.Cu") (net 4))
 (segment (start 25.04 6.9183) (end 27.89 9.7683) (width 1) (layer "B.Cu") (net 4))
 (segment (start 27.89 22.8917) (end 26.5017 22.8917) (width 1) (layer "B.Cu") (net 4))
 (segment (start 27.89 11.62) (end 27.89 9.7683) (width 1) (layer "B.Cu") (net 4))
 (segment (start 23.4273 26.4) (end 22.4 26.4) (width 1) (layer "B.Cu") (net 4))
 (segment (start 14.7 34.04) (end 11.18 34.04) (width 1) (layer "B.Cu") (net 4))
 (segment (start 7.7 30.56) (end 10.94 27.32) (width 1) (layer "B.Cu") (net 4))
 (segment (start 22.26 5.7017) (end 25.04 5.7017) (width 1) (layer "B.Cu") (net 4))
 (segment (start 22.7338 30.0738) (end 22.4 30.0738) (width 1) (layer "B.Cu") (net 4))
 (segment (start 25.04 5.7017) (end 25.04 6.9183) (width 1) (layer "B.Cu") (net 4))
 (segment (start 21.4217 7.6417) (end 22.4 8.62) (width 1) (layer "B.Cu") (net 4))
 (segment (start 10.94 27.32) (end 10.94 26.9) (width 1) (layer "B.Cu") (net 4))
 (segment (start 21.4217 6.54) (end 22.26 5.7017) (width 1) (layer "B.Cu") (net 4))
 (segment (start 26.5017 23.3256) (end 23.4273 26.4) (width 1) (layer "B.Cu") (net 4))
 (segment (start 22.4 30.0738) (end 18.6662 30.0738) (width 1) (layer "B.Cu") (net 4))
 (segment (start 18.6662 30.0738) (end 14.7 34.04) (width 1) (layer "B.Cu") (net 4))
 (segment (start 21.4217 6.54) (end 21.4217 7.6417) (width 1) (layer "B.Cu") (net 4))
 (segment (start 25.35 32.69) (end 22.7338 30.0738) (width 1) (layer "B.Cu") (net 4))
 (segment (start 26.5017 22.8917) (end 26.5017 23.3256) (width 1) (layer "B.Cu") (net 4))
 (segment (start 27.89 21.04) (end 27.89 22.8917) (width 1) (layer "B.Cu") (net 4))
 (segment (start 25.04 3.4) (end 25.04 5.7017) (width 1) (layer "B.Cu") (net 4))
 (segment (start 22.4 26.4) (end 22.4 30.0738) (width 1) (layer "B.Cu") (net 4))
 (segment (start 9.2 25.16) (end 9.2 24.32) (width 1) (layer "B.Cu") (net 4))
 (segment (start 14.2 9.08) (end 11.7 9.08) (width 1) (layer "B.Cu") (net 5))
 (segment (start 16.7 9.08) (end 14.2 9.08) (width 1) (layer "B.Cu") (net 5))
 (segment (start 16.7 9.08) (end 19.32 9.08) (width 1) (layer "B.Cu") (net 5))
 (segment (start 22.5 3.4) (end 22.0217 3.4) (width 1) (layer "B.Cu") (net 3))
 (segment (start 22.0217 3.4) (end 21.4217 4) (width 1) (layer "B.Cu") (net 3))
 (segment (start 19.32 4) (end 21.4217 4) (width 1) (layer "B.Cu") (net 3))
 (segment (start 22.7983 14.16) (end 22.7983 22.69) (width 0.6) (layer "B.Cu") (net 7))
 (segment (start 16.7 16.7) (end 16.7 15.0498) (width 0.6) (layer "B.Cu") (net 7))
 (segment (start 16.7 15.0498) (end 17.4933 14.2565) (width 0.6) (layer "B.Cu") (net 7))
 (segment (start 27.89 14.16) (end 25.8883 14.16) (width 0.6) (layer "B.Cu") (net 7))
 (segment (start 24.3 22.69) (end 22.7983 22.69) (width 0.6) (layer "B.Cu") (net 7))
 (segment (start 19.32 14.16) (end 17.4933 14.16) (width 0.6) (layer "B.Cu") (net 7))
 (segment (start 25.8883 14.16) (end 22.7983 14.16) (width 0.6) (layer "B.Cu") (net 7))
 (segment (start 22.7983 14.16) (end 21.1467 14.16) (width 0.6) (layer "B.Cu") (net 7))
 (segment (start 17.4933 14.2565) (end 17.4933 14.16) (width 0.6) (layer "B.Cu") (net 7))
 (segment (start 19.32 14.16) (end 21.1467 14.16) (width 0.6) (layer "B.Cu") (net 7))
 (segment (start 25 11.62) (end 19.32 11.62) (width 0.6) (layer "B.Cu") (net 6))
 (segment (start 25 19.24) (end 25.1483 19.24) (width 0.6) (layer "B.Cu") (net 20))
 (segment (start 27.89 18.5) (end 25.8883 18.5) (width 0.6) (layer "B.Cu") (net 20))
 (segment (start 25.1483 19.24) (end 25.8883 18.5) (width 0.6) (layer "B.Cu") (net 20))
 (segment (start 6.7 4) (end 4.08 4) (width 0.6) (layer "B.Cu") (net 1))
 (segment (start 6.7965 7.4298) (end 5.9067 6.54) (width 0.6) (layer "B.Cu") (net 2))
 (segment (start 4.08 6.54) (end 5.9067 6.54) (width 0.6) (layer "B.Cu") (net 2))
 (segment (start 8.5444 6.54) (end 7.6546 7.4298) (width 0.6) (layer "B.Cu") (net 2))
 (segment (start 7.6546 7.4298) (end 6.7965 7.4298) (width 0.6) (layer "B.Cu") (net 2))
 (segment (start 9.2 6.54) (end 8.5444 6.54) (width 0.6) (layer "B.Cu") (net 2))
 (segment (start 6.7 11.62) (end 9.2 14.12) (width 0.6) (layer "B.Cu") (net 13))
 (segment (start 8.66 14.7) (end 9.2 14.16) (width 0.6) (layer "B.Cu") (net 13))
 (segment (start 9.2 14.12) (end 9.2 14.16) (width 0.6) (layer "B.Cu") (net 13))
 (segment (start 6.7 14.7) (end 8.66 14.7) (width 0.6) (layer "B.Cu") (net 13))
 (segment (start 4.46 25.5) (end 4.46 24.56) (width 0.6) (layer "B.Cu") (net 9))
 (segment (start 4.46 24.56) (end 6.7 22.32) (width 0.6) (layer "B.Cu") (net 9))
 (segment (start 4.46 25.5) (end 5.86 26.9) (width 0.6) (layer "B.Cu") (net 9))
 (segment (start 3.3 25.5) (end 4.46 25.5) (width 0.6) (layer "B.Cu") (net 9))
 (segment (start 5.7 35.66) (end 7.68 35.66) (width 0.6) (layer "B.Cu") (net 17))
 (segment (start 3.3 35.66) (end 5.7 35.66) (width 0.6) (layer "B.Cu") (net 17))
 (segment (start 7.68 35.66) (end 7.7 35.64) (width 0.6) (layer "B.Cu") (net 17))
 (segment (start 5.7 35.66) (end 5.7 41.5) (width 0.6) (layer "B.Cu") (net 17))
 (segment (start 7.7 39.5983) (end 9.2017 39.5983) (width 0.6) (layer "B.Cu") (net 19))
 (segment (start 7.7 41.5) (end 7.7 39.5983) (width 0.6) (layer "B.Cu") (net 19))
 (segment (start 9.2017 39.5983) (end 10.7 38.1) (width 0.6) (layer "B.Cu") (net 19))
 (segment (start 18.2 43.1) (end 10.7 43.1) (width 0.6) (layer "B.Cu") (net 10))
 (segment (start 20.1 40) (end 20.7 40.6) (width 0.6) (layer "B.Cu") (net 10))
 (segment (start 20.1 32.08) (end 20.1 40) (width 0.6) (layer "B.Cu") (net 10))
 (segment (start 20.7 40.6) (end 18.2 43.1) (width 0.6) (layer "B.Cu") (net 10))
 (segment (start 20.7 40.6) (end 25.06 40.6) (width 0.6) (layer "B.Cu") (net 10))
 (segment (start 25.06 40.6) (end 25.35 40.31) (width 0.6) (layer "B.Cu") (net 10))
 (segment (start 16.7 26.86) (end 19.96 26.86) (width 0.6) (layer "B.Cu") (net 14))
 (segment (start 19.96 26.86) (end 20.1 27) (width 0.6) (layer "B.Cu") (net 14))
 (segment (start 16.7 19.24) (end 14.2 19.24) (width 0.6) (layer "B.Cu") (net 8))
 (segment (start 14.7 26.2572) (end 16.7 24.2572) (width 0.6) (layer "B.Cu") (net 8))
 (segment (start 16.7 19.24) (end 19.32 19.24) (width 0.6) (layer "B.Cu") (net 8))
 (segment (start 9.2 16.7) (end 11.7 16.7) (width 0.6) (layer "B.Cu") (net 8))
 (segment (start 14.7 28.96) (end 14.7 26.2572) (width 0.6) (layer "B.Cu") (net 8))
 (segment (start 11.7 16.7) (end 14.2 16.7) (width 0.6) (layer "B.Cu") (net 8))
 (segment (start 16.7 24.2572) (end 16.7 19.24) (width 0.6) (layer "B.Cu") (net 8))
 (segment (start 14.2 19.24) (end 14.2 16.7) (width 0.6) (layer "B.Cu") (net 8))
 (segment (start 11.7 14.16) (end 11.7 16.7) (width 0.6) (layer "B.Cu") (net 8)))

